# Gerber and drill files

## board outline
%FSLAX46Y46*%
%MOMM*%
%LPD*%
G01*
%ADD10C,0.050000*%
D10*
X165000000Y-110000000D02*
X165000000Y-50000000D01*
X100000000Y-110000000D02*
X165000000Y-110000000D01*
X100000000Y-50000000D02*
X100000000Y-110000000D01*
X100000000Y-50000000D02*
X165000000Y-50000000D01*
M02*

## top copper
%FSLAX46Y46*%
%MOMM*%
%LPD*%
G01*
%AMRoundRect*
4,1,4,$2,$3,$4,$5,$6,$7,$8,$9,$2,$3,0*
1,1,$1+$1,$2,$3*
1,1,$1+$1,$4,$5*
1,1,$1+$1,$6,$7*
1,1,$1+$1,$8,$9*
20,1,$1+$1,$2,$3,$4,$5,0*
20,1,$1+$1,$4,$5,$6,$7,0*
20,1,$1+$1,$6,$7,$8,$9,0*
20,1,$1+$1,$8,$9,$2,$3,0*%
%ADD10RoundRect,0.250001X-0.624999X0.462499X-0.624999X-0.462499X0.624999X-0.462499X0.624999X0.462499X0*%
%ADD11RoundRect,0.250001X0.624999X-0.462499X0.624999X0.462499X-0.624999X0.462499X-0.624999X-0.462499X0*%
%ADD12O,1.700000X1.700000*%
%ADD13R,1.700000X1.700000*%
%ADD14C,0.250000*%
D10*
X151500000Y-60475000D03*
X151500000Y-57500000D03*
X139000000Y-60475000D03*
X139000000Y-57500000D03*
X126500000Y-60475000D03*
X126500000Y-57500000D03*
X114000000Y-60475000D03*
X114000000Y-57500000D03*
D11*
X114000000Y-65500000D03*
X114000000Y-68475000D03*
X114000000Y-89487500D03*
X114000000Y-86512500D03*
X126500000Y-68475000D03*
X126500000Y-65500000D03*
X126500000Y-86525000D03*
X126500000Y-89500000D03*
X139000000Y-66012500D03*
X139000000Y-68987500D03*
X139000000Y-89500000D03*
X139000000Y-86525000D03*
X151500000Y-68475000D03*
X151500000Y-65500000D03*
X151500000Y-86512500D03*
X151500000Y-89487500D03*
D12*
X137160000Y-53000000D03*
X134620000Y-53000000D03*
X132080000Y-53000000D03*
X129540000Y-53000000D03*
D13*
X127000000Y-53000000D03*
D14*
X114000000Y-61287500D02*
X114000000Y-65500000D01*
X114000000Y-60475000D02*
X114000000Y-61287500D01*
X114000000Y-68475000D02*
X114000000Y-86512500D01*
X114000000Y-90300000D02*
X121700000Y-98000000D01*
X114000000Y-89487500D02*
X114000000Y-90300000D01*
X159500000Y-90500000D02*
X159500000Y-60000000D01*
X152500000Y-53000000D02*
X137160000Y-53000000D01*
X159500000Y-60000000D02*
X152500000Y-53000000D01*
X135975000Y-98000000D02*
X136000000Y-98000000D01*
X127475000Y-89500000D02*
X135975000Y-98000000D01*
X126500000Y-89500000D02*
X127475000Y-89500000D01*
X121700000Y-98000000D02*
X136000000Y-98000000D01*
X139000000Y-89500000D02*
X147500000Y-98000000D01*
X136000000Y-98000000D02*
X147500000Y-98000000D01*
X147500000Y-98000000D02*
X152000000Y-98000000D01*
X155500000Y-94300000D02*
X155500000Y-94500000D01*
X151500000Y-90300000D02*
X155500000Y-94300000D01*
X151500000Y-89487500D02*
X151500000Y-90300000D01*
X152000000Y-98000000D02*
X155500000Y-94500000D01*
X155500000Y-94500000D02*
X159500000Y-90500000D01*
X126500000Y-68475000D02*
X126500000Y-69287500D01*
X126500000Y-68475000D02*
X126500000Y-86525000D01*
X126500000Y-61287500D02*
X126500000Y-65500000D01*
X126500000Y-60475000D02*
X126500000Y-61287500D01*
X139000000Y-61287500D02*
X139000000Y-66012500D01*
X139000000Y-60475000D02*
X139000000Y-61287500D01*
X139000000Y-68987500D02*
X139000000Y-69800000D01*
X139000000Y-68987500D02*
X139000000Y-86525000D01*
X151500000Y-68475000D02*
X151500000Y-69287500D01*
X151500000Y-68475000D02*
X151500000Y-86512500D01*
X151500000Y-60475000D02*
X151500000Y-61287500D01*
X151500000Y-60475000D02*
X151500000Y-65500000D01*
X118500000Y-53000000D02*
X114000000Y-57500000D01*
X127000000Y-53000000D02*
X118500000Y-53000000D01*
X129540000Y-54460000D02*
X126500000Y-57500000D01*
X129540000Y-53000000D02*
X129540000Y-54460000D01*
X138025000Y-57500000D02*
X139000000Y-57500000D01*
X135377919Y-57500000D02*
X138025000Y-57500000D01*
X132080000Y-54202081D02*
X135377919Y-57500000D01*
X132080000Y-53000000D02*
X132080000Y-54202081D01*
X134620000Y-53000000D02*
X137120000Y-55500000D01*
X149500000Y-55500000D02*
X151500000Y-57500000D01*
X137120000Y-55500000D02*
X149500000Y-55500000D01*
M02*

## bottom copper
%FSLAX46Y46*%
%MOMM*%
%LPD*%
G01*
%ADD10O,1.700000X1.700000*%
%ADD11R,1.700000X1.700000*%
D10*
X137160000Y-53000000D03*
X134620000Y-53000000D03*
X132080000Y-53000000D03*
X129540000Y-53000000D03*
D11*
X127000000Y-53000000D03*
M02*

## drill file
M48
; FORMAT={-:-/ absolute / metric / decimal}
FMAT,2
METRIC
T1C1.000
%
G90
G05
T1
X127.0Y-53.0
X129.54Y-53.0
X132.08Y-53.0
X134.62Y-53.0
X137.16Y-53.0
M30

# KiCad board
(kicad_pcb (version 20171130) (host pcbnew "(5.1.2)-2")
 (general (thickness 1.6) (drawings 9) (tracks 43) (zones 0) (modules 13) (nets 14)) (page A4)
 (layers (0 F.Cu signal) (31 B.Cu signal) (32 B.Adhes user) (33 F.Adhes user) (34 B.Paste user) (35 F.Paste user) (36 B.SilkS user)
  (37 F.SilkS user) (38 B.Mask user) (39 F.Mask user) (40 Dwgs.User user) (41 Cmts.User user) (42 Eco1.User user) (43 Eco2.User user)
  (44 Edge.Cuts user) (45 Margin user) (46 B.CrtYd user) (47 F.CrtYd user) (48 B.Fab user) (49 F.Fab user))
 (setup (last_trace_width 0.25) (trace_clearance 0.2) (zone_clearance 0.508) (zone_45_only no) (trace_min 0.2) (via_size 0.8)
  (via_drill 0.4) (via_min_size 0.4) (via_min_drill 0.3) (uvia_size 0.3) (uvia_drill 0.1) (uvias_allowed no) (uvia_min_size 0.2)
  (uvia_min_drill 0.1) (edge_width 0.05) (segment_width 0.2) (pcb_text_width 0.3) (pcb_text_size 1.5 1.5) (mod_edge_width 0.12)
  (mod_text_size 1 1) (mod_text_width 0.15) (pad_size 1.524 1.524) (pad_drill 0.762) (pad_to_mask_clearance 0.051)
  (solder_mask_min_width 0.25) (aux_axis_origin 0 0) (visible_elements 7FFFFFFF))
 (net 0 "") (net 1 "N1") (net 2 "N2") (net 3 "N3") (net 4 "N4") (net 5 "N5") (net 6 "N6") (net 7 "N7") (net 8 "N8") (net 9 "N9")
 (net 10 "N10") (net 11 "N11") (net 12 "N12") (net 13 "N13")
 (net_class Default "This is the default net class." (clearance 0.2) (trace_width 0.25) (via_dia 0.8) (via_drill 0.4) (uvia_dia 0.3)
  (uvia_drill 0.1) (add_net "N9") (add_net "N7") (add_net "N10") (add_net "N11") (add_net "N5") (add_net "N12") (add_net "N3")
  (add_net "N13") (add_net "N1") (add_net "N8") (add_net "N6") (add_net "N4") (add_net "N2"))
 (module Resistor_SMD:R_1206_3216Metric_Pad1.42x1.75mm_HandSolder (layer F.Cu) (at 151.5 58.9875 270)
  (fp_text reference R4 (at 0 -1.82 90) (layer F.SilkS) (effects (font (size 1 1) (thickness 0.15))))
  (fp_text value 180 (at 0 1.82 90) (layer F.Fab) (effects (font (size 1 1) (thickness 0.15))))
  (pad 2 smd roundrect (at 1.4875 0 270) (size 1.425 1.75) (layers F.Cu F.Paste F.Mask) (roundrect_rratio 0.175439) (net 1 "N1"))
  (pad 1 smd roundrect (at -1.4875 0 270) (size 1.425 1.75) (layers F.Cu F.Paste F.Mask) (roundrect_rratio 0.175439) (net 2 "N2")))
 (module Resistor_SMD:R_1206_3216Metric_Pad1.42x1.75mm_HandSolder (layer F.Cu) (at 139 58.9875 270)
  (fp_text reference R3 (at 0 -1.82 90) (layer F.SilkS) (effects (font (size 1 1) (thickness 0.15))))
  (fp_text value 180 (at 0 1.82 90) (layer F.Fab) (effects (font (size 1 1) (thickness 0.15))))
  (pad 2 smd roundrect (at 1.4875 0 270) (size 1.425 1.75) (layers F.Cu F.Paste F.Mask) (roundrect_rratio 0.175439) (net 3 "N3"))
  (pad 1 smd roundrect (at -1.4875 0 270) (size 1.425 1.75) (layers F.Cu F.Paste F.Mask) (roundrect_rratio 0.175439) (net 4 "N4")))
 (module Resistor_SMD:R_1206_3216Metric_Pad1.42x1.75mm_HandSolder (layer F.Cu) (at 126.5 58.9875 270)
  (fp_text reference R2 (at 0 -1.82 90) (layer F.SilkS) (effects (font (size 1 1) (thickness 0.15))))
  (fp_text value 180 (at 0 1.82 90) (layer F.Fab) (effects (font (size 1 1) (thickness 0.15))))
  (pad 2 smd roundrect (at 1.4875 0 270) (size 1.425 1.75) (layers F.Cu F.Paste F.Mask) (roundrect_rratio 0.175439) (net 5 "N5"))
  (pad 1 smd roundrect (at -1.4875 0 270) (size 1.425 1.75) (layers F.Cu F.Paste F.Mask) (roundrect_rratio 0.175439) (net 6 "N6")))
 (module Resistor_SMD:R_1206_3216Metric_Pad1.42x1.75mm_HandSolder (layer F.Cu) (at 114 58.9875 270)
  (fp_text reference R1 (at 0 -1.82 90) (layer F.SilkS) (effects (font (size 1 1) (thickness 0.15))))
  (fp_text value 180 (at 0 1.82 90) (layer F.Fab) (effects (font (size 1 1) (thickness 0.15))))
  (pad 2 smd roundrect (at 1.4875 0 270) (size 1.425 1.75) (layers F.Cu F.Paste F.Mask) (roundrect_rratio 0.175439) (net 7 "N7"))
  (pad 1 smd roundrect (at -1.4875 0 270) (size 1.425 1.75) (layers F.Cu F.Paste F.Mask) (roundrect_rratio 0.175439) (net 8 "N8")))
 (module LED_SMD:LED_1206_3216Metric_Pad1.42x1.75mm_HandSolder (layer F.Cu) (at 114 66.9875 90)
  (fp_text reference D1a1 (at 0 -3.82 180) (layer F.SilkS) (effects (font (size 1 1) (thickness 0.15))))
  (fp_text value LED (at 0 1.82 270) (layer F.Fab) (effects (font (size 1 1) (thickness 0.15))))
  (pad 2 smd roundrect (at 1.4875 0 90) (size 1.425 1.75) (layers F.Cu F.Paste F.Mask) (roundrect_rratio 0.175439) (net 7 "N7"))
  (pad 1 smd roundrect (at -1.4875 0 90) (size 1.425 1.75) (layers F.Cu F.Paste F.Mask) (roundrect_rratio 0.175439) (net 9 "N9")))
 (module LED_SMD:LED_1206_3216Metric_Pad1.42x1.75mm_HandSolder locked (layer F.Cu) (at 114 88 90)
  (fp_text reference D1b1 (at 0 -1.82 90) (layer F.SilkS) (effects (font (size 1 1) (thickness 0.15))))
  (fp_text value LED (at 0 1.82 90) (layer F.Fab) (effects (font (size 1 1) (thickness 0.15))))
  (pad 1 smd roundrect (at -1.4875 0 90) (size 1.425 1.75) (layers F.Cu F.Paste F.Mask) (roundrect_rratio 0.175439) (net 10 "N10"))
  (pad 2 smd roundrect (at 1.4875 0 90) (size 1.425 1.75) (layers F.Cu F.Paste F.Mask) (roundrect_rratio 0.175439) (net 9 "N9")))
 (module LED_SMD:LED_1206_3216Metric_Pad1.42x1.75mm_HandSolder (layer F.Cu) (at 126.5 66.9875 90)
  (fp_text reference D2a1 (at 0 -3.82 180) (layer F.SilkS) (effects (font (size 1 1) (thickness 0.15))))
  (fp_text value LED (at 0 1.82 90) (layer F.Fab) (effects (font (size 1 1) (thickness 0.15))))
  (pad 1 smd roundrect (at -1.4875 0 90) (size 1.425 1.75) (layers F.Cu F.Paste F.Mask) (roundrect_rratio 0.175439) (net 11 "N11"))
  (pad 2 smd roundrect (at 1.4875 0 90) (size 1.425 1.75) (layers F.Cu F.Paste F.Mask) (roundrect_rratio 0.175439) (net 5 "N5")))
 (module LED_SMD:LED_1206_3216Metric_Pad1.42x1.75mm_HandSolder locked (layer F.Cu) (at 126.5 88.0125 90)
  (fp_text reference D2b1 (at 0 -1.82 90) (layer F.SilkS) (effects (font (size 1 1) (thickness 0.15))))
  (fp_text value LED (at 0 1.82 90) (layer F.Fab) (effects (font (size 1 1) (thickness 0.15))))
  (pad 2 smd roundrect (at 1.4875 0 90) (size 1.425 1.75) (layers F.Cu F.Paste F.Mask) (roundrect_rratio 0.175439) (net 11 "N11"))
  (pad 1 smd roundrect (at -1.4875 0 90) (size 1.425 1.75) (layers F.Cu F.Paste F.Mask) (roundrect_rratio 0.175439) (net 10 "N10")))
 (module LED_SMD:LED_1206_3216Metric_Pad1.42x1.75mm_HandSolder (layer F.Cu) (at 139 67.5 90)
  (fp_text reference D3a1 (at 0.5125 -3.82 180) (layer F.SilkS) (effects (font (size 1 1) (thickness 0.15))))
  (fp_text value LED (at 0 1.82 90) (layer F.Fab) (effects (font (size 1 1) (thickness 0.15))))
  (pad 2 smd roundrect (at 1.4875 0 90) (size 1.425 1.75) (layers F.Cu F.Paste F.Mask) (roundrect_rratio 0.175439) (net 3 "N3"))
  (pad 1 smd roundrect (at -1.4875 0 90) (size 1.425 1.75) (layers F.Cu F.Paste F.Mask) (roundrect_rratio 0.175439) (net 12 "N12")))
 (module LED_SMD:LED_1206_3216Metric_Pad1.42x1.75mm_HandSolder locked (layer F.Cu) (at 139 88.0125 90)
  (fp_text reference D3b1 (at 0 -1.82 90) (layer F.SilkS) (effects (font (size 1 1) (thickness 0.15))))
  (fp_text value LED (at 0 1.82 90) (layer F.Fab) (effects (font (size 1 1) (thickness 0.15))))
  (pad 1 smd roundrect (at -1.4875 0 90) (size 1.425 1.75) (layers F.Cu F.Paste F.Mask) (roundrect_rratio 0.175439) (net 10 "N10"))
  (pad 2 smd roundrect (at 1.4875 0 90) (size 1.425 1.75) (layers F.Cu F.Paste F.Mask) (roundrect_rratio 0.175439) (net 12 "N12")))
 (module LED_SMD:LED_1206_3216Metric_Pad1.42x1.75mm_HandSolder (layer F.Cu) (at 151.5 66.9875 90)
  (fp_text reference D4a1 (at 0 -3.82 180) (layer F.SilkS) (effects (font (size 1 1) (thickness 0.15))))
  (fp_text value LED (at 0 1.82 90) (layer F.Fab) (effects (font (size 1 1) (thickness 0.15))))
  (pad 1 smd roundrect (at -1.4875 0 90) (size 1.425 1.75) (layers F.Cu F.Paste F.Mask) (roundrect_rratio 0.175439) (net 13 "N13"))
  (pad 2 smd roundrect (at 1.4875 0 90) (size 1.425 1.75) (layers F.Cu F.Paste F.Mask) (roundrect_rratio 0.175439) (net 1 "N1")))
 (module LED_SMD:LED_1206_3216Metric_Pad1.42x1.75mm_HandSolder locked (layer F.Cu) (at 151.5 88 90)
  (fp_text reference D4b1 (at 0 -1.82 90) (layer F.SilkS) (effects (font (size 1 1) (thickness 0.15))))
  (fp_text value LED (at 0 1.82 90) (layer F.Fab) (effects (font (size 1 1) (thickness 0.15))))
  (pad 2 smd roundrect (at 1.4875 0 90) (size 1.425 1.75) (layers F.Cu F.Paste F.Mask) (roundrect_rratio 0.175439) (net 13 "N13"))
  (pad 1 smd roundrect (at -1.4875 0 90) (size 1.425 1.75) (layers F.Cu F.Paste F.Mask) (roundrect_rratio 0.175439) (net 10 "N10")))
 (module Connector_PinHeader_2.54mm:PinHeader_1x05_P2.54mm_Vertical (layer F.Cu) (at 127 53 90)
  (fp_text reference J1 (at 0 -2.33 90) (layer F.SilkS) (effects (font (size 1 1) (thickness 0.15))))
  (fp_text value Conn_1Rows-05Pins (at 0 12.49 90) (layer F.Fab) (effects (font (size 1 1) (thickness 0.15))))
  (pad 5 thru_hole oval (at 0 10.16 90) (size 1.7 1.7) (drill 1) (layers *.Cu *.Mask) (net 10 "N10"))
  (pad 4 thru_hole oval (at 0 7.62 90) (size 1.7 1.7) (drill 1) (layers *.Cu *.Mask) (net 2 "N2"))
  (pad 3 thru_hole oval (at 0 5.08 90) (size 1.7 1.7) (drill 1) (layers *.Cu *.Mask) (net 4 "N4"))
  (pad 2 thru_hole oval (at 0 2.54 90) (size 1.7 1.7) (drill 1) (layers *.Cu *.Mask) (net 6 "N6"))
  (pad 1 thru_hole rect (at 0 0 90) (size 1.7 1.7) (drill 1) (layers *.Cu *.Mask) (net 8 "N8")))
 (gr_line (start 165 110) (end 165 50) (layer Edge.Cuts) (width 0.05))
 (gr_line (start 100 110) (end 165 110) (layer Edge.Cuts) (width 0.05))
 (gr_line (start 100 50) (end 100 110) (layer Edge.Cuts) (width 0.05))
 (gr_line (start 100 50) (end 165 50) (layer Edge.Cuts) (width 0.05))
 (segment (start 114 61.2875) (end 114 65.5) (width 0.25) (layer F.Cu) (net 7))
 (segment (start 114 60.475) (end 114 61.2875) (width 0.25) (layer F.Cu) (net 7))
 (segment (start 114 68.475) (end 114 86.5125) (width 0.25) (layer F.Cu) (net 9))
 (segment (start 114 90.3) (end 121.7 98) (width 0.25) (layer F.Cu) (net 10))
 (segment (start 114 89.4875) (end 114 90.3) (width 0.25) (layer F.Cu) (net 10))
 (segment (start 159.5 90.5) (end 159.5 60) (width 0.25) (layer F.Cu) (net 10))
 (segment (start 152.5 53) (end 137.16 53) (width 0.25) (layer F.Cu) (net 10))
 (segment (start 159.5 60) (end 152.5 53) (width 0.25) (layer F.Cu) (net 10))
 (segment (start 135.975 98) (end 136 98) (width 0.25) (layer F.Cu) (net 10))
 (segment (start 127.475 89.5) (end 135.975 98) (width 0.25) (layer F.Cu) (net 10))
 (segment (start 126.5 89.5) (end 127.475 89.5) (width 0.25) (layer F.Cu) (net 10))
 (segment (start 121.7 98) (end 136 98) (width 0.25) (layer F.Cu) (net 10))
 (segment (start 139 89.5) (end 147.5 98) (width 0.25) (layer F.Cu) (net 10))
 (segment (start 136 98) (end 147.5 98) (width 0.25) (layer F.Cu) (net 10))
 (segment (start 147.5 98) (end 152 98) (width 0.25) (layer F.Cu) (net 10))
 (segment (start 155.5 94.3) (end 155.5 94.5) (width 0.25) (layer F.Cu) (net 10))
 (segment (start 151.5 90.3) (end 155.5 94.3) (width 0.25) (layer F.Cu) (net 10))
 (segment (start 151.5 89.4875) (end 151.5 90.3) (width 0.25) (layer F.Cu) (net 10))
 (segment (start 152 98) (end 155.5 94.5) (width 0.25) (layer F.Cu) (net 10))
 (segment (start 155.5 94.5) (end 159.5 90.5) (width 0.25) (layer F.Cu) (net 10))
 (segment (start 126.5 68.475) (end 126.5 69.2875) (width 0.25) (layer F.Cu) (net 11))
 (segment (start 126.5 68.475) (end 126.5 86.525) (width 0.25) (layer F.Cu) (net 11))
 (segment (start 126.5 61.2875) (end 126.5 65.5) (width 0.25) (layer F.Cu) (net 5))
 (segment (start 126.5 60.475) (end 126.5 61.2875) (width 0.25) (layer F.Cu) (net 5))
 (segment (start 139 61.2875) (end 139 66.0125) (width 0.25) (layer F.Cu) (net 3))
 (segment (start 139 60.475) (end 139 61.2875) (width 0.25) (layer F.Cu) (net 3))
 (segment (start 139 68.9875) (end 139 69.8) (width 0.25) (layer F.Cu) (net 12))
 (segment (start 139 68.9875) (end 139 86.525) (width 0.25) (layer F.Cu) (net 12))
 (segment (start 151.5 68.475) (end 151.5 69.2875) (width 0.25) (layer F.Cu) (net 13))
 (segment (start 151.5 68.475) (end 151.5 86.5125) (width 0.25) (layer F.Cu) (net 13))
 (segment (start 151.5 60.475) (end 151.5 61.2875) (width 0.25) (layer F.Cu) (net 1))
 (segment (start 151.5 60.475) (end 151.5 65.5) (width 0.25) (layer F.Cu) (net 1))
 (segment (start 118.5 53) (end 114 57.5) (width 0.25) (layer F.Cu) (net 8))
 (segment (start 127 53) (end 118.5 53) (width 0.25) (layer F.Cu) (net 8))
 (segment (start 129.54 54.46) (end 126.5 57.5) (width 0.25) (layer F.Cu) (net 6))
 (segment (start 129.54 53) (end 129.54 54.46) (width 0.25) (layer F.Cu) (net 6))
 (segment (start 138.025 57.5) (end 139 57.5) (width 0.25) (layer F.Cu) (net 4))
 (segment (start 135.377919 57.5) (end 138.025 57.5) (width 0.25) (layer F.Cu) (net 4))
 (segment (start 132.08 54.202081) (end 135.377919 57.5) (width 0.25) (layer F.Cu) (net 4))
 (segment (start 132.08 53) (end 132.08 54.202081) (width 0.25) (layer F.Cu) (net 4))
 (segment (start 134.62 53) (end 137.12 55.5) (width 0.25) (layer F.Cu) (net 2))
 (segment (start 149.5 55.5) (end 151.5 57.5) (width 0.25) (layer F.Cu) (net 2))
 (segment (start 137.12 55.5) (end 149.5 55.5) (width 0.25) (layer F.Cu) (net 2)))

